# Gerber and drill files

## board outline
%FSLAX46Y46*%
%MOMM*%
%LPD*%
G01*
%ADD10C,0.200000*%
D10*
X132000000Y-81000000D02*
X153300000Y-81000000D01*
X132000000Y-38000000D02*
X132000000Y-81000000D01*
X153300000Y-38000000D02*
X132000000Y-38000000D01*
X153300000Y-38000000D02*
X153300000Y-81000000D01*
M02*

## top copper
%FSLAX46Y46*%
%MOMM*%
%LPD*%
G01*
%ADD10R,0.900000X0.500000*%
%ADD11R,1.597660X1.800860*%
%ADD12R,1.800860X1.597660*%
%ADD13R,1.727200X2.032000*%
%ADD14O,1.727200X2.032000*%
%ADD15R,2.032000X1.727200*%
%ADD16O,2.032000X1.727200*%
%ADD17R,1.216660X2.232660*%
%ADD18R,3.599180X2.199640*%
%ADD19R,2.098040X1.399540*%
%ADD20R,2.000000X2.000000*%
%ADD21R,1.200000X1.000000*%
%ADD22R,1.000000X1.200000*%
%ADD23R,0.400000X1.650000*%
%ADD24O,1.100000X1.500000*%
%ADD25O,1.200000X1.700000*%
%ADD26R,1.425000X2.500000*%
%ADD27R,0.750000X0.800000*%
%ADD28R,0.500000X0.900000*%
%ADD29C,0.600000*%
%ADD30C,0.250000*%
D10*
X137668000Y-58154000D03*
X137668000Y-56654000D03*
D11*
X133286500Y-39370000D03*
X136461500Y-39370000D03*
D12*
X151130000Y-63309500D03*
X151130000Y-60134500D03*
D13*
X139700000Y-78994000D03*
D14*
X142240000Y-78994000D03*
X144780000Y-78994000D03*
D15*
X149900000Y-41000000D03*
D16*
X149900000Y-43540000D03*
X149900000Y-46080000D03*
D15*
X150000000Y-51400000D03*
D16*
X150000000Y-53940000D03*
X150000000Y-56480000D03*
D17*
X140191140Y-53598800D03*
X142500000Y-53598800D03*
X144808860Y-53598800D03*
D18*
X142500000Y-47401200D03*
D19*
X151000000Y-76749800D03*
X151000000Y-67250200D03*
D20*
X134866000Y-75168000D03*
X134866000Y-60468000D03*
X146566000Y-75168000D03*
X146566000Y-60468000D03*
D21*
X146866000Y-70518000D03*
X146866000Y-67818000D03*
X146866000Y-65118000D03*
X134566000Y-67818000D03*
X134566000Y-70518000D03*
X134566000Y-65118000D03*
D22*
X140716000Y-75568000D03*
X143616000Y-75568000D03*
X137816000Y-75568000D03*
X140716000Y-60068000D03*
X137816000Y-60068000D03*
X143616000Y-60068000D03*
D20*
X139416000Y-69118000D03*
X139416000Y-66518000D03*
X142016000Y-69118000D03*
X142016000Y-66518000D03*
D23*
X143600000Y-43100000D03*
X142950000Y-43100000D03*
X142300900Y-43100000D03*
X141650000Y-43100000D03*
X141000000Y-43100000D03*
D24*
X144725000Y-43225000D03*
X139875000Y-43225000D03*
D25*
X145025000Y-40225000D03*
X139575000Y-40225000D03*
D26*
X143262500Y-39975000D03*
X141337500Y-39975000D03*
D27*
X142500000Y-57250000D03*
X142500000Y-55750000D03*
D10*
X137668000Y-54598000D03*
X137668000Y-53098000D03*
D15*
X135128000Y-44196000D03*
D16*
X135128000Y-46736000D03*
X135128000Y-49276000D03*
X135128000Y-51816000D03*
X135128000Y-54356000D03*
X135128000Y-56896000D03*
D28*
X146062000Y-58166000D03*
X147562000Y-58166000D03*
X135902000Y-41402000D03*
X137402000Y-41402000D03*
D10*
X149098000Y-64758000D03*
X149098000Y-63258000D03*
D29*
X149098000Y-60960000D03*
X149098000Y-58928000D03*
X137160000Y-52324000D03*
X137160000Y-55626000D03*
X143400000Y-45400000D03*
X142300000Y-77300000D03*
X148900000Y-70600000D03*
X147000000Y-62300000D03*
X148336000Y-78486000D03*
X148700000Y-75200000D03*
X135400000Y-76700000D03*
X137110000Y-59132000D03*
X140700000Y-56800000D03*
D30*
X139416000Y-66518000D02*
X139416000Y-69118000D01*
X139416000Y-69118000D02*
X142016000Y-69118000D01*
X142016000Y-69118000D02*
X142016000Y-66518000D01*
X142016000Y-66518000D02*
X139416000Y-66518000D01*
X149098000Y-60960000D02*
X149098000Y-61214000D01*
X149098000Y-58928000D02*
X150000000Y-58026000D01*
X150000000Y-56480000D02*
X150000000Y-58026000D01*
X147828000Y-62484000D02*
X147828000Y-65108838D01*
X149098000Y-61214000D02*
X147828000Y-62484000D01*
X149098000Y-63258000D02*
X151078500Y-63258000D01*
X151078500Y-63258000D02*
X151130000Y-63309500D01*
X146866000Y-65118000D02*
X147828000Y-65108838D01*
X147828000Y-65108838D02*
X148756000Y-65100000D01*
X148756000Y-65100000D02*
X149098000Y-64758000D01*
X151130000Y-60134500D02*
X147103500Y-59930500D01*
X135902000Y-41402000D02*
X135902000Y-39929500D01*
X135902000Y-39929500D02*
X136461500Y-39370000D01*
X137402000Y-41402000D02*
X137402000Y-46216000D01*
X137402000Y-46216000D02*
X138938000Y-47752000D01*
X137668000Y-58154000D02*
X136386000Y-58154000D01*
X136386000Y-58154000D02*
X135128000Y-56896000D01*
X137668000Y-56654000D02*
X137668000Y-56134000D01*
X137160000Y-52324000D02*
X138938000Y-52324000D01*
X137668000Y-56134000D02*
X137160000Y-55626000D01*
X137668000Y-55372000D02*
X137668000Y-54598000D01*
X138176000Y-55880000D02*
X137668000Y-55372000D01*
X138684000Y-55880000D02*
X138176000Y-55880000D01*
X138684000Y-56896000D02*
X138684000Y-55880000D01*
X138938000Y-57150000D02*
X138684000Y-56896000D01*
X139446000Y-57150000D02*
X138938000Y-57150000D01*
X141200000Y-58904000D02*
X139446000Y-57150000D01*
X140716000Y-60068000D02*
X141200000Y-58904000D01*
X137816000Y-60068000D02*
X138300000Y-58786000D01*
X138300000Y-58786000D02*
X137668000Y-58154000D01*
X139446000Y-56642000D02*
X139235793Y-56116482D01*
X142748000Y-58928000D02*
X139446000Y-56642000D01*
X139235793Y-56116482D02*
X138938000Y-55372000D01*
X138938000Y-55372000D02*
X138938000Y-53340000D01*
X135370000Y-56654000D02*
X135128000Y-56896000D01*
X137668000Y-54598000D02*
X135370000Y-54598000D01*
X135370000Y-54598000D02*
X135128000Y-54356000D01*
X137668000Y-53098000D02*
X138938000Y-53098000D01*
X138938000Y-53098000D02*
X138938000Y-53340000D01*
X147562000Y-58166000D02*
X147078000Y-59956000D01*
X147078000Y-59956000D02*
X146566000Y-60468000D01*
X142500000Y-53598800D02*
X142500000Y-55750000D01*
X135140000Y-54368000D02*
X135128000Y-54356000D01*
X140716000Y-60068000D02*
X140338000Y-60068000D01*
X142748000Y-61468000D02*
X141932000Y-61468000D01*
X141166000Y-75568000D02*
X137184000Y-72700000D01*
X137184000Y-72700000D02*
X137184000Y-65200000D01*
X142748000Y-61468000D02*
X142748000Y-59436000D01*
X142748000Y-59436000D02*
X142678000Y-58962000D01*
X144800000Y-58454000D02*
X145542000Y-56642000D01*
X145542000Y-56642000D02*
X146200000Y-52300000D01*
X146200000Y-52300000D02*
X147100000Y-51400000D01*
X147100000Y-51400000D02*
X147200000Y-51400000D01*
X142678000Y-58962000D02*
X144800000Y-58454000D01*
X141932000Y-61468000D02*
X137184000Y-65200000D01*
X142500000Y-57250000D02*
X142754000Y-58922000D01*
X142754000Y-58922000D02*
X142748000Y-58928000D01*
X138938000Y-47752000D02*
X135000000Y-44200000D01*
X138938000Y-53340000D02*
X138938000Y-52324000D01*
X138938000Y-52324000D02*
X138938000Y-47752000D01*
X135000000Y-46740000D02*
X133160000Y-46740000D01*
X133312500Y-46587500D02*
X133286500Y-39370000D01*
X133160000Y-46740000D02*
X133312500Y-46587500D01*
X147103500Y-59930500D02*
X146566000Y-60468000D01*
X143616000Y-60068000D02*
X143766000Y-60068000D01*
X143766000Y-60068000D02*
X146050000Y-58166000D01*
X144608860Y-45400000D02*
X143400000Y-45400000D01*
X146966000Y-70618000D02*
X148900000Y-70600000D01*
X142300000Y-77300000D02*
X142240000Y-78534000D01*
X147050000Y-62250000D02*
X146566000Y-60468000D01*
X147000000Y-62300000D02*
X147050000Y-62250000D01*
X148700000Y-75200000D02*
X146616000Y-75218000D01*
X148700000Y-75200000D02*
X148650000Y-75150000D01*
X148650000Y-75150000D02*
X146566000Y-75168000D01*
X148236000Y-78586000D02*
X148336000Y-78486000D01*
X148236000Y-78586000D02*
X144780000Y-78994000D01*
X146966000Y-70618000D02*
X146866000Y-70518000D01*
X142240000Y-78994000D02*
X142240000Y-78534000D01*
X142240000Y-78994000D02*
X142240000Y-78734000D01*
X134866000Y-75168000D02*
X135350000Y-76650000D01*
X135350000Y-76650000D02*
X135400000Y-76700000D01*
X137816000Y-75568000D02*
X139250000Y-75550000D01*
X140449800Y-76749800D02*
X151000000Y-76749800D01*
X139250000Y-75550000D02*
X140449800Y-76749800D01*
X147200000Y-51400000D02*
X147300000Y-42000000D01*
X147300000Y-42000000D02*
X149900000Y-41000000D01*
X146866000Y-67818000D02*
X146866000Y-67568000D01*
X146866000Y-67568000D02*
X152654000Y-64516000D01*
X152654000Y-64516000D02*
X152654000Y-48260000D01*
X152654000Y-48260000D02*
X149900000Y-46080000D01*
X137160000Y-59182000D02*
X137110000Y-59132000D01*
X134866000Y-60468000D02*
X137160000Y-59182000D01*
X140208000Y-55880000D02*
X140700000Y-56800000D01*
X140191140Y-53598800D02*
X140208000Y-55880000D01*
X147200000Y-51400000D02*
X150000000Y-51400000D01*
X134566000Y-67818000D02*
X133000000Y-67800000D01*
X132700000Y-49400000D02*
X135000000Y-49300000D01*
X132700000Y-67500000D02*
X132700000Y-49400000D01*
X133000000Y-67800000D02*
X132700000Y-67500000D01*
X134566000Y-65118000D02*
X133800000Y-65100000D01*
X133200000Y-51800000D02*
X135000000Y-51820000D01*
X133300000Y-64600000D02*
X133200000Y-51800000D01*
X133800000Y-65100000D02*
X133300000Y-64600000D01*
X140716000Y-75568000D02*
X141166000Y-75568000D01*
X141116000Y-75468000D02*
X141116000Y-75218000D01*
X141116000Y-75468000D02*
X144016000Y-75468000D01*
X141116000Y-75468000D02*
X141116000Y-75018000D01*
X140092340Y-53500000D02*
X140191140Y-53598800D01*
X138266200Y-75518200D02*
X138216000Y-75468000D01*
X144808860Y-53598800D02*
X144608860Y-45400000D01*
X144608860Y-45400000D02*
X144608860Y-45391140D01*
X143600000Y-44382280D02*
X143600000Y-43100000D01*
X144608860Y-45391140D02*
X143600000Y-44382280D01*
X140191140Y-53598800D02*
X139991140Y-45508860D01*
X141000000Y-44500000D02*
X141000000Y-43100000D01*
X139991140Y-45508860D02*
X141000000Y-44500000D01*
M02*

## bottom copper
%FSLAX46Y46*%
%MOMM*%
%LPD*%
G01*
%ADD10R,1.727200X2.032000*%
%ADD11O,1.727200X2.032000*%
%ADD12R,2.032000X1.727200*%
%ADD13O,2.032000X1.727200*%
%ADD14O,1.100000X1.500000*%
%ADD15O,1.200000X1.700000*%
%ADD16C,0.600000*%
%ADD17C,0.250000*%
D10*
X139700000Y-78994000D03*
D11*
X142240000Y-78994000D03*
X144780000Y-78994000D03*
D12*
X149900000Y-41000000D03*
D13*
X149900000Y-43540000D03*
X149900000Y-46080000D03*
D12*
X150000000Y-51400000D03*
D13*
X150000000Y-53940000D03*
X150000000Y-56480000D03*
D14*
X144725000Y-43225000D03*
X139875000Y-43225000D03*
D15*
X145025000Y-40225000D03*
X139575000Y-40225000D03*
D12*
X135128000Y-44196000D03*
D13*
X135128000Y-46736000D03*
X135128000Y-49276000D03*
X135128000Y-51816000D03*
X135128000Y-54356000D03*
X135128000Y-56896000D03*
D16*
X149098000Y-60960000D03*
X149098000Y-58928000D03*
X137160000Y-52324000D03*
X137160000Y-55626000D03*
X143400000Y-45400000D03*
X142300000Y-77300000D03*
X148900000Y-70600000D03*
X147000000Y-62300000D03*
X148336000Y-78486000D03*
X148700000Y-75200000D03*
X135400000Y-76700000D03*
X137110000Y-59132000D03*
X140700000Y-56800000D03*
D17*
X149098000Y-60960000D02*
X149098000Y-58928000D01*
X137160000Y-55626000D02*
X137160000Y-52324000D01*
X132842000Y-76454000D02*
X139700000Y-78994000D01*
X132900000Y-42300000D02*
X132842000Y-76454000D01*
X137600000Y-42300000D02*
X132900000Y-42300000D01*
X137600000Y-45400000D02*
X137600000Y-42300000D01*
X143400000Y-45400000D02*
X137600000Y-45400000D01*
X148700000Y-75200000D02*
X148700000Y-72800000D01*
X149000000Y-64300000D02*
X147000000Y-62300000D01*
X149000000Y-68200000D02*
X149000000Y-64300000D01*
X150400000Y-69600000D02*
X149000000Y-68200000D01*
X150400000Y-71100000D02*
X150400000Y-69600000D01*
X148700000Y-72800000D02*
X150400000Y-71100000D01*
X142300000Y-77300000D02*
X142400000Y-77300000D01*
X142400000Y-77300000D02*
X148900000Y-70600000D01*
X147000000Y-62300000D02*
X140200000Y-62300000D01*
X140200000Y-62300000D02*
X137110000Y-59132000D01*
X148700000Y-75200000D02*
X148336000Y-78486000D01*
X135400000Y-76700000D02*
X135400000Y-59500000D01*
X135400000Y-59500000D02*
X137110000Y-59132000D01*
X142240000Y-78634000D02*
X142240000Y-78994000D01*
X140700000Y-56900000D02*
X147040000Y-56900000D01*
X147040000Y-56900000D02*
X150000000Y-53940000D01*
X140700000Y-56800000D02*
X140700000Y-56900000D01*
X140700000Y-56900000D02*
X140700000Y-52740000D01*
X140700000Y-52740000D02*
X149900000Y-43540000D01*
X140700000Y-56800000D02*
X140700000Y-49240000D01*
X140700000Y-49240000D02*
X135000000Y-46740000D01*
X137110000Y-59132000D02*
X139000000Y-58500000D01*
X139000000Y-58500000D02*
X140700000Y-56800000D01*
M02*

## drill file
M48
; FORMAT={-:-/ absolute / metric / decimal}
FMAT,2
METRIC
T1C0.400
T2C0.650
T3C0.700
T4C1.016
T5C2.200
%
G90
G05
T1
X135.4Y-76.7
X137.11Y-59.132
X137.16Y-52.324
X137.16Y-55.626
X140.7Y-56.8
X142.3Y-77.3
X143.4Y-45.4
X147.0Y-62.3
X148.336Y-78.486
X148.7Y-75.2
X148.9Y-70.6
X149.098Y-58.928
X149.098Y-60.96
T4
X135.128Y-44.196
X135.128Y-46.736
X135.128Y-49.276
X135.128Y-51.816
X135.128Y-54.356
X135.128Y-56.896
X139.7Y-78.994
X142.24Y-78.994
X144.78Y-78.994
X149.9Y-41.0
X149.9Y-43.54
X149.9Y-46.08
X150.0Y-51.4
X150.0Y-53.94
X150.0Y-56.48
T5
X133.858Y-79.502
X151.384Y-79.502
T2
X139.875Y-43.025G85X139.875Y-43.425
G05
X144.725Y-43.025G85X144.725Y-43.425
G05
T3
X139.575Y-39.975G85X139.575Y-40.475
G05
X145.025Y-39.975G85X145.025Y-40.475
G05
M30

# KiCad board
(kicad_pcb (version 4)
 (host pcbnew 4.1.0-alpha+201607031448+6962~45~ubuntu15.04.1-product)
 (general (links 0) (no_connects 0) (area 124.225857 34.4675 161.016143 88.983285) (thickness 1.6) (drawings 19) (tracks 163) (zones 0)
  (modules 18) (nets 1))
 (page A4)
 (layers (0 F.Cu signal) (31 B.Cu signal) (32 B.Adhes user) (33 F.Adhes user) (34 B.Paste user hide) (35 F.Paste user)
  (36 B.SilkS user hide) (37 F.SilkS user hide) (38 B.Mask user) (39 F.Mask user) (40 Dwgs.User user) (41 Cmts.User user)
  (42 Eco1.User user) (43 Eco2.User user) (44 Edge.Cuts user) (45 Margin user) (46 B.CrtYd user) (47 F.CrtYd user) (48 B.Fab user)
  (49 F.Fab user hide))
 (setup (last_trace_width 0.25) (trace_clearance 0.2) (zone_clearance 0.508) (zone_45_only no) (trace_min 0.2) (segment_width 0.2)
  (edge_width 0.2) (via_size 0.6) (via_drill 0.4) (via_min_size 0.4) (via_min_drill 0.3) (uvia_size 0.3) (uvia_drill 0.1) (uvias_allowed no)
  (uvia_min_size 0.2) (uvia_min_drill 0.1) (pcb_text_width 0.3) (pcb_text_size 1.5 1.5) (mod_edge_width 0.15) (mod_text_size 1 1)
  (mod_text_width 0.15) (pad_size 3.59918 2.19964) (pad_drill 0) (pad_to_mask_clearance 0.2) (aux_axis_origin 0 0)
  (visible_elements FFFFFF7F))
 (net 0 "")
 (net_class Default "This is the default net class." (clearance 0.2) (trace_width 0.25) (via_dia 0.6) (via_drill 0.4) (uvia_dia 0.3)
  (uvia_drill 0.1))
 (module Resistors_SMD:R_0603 (layer F.Cu) (at 137.668 57.404 90)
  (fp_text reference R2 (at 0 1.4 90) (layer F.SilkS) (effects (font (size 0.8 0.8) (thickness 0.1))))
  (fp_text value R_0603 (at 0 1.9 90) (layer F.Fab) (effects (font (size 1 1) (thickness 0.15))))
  (pad 1 smd rect (at -0.75 0 90) (size 0.5 0.9) (layers F.Cu F.Paste F.Mask))
  (pad 2 smd rect (at 0.75 0 90) (size 0.5 0.9) (layers F.Cu F.Paste F.Mask)))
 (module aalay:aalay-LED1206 (layer F.Cu) (at 134.874 39.37)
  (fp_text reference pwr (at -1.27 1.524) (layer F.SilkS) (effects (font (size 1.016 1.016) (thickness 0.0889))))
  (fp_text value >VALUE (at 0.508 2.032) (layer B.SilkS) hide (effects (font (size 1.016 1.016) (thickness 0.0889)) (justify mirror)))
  (pad A smd rect (at -1.5875 0) (size 1.59766 1.80086) (layers F.Cu F.Paste F.Mask))
  (pad K smd rect (at 1.5875 0) (size 1.59766 1.80086) (layers F.Cu F.Paste F.Mask)))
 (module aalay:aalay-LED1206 (layer F.Cu) (at 151.13 61.722 90)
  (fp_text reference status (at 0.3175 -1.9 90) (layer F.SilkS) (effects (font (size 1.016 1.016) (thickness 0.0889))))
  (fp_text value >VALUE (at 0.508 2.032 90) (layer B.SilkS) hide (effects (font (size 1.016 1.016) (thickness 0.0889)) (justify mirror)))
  (pad A smd rect (at -1.5875 0 90) (size 1.59766 1.80086) (layers F.Cu F.Paste F.Mask))
  (pad K smd rect (at 1.5875 0 90) (size 1.59766 1.80086) (layers F.Cu F.Paste F.Mask)))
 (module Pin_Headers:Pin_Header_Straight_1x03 (layer F.Cu) (at 139.7 78.994 90)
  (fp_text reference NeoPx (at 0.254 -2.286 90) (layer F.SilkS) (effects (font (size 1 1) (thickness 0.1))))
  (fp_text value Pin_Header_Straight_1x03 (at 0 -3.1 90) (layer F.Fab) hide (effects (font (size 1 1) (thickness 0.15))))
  (pad 1 thru_hole rect (at 0 0 90) (size 2.032 1.7272) (drill 1.016) (layers *.Cu *.Mask F.SilkS))
  (pad 2 thru_hole oval (at 0 2.54 90) (size 2.032 1.7272) (drill 1.016) (layers *.Cu *.Mask F.SilkS))
  (pad 3 thru_hole oval (at 0 5.08 90) (size 2.032 1.7272) (drill 1.016) (layers *.Cu *.Mask F.SilkS)))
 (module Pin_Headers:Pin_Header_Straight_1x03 (layer F.Cu) (at 149.9 41)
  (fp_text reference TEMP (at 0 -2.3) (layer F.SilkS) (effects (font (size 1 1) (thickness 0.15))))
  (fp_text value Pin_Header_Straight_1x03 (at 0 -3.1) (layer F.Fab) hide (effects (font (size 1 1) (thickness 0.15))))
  (pad 1 thru_hole rect (at 0 0) (size 2.032 1.7272) (drill 1.016) (layers *.Cu *.Mask F.SilkS))
  (pad 2 thru_hole oval (at 0 2.54) (size 2.032 1.7272) (drill 1.016) (layers *.Cu *.Mask F.SilkS))
  (pad 3 thru_hole oval (at 0 5.08) (size 2.032 1.7272) (drill 1.016) (layers *.Cu *.Mask F.SilkS)))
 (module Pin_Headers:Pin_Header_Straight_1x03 (layer F.Cu) (at 150 51.4)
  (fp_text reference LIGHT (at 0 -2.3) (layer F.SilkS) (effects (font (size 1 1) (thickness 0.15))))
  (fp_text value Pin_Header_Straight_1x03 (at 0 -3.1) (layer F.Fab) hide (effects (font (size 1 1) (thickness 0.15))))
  (pad 1 thru_hole rect (at 0 0) (size 2.032 1.7272) (drill 1.016) (layers *.Cu *.Mask F.SilkS))
  (pad 2 thru_hole oval (at 0 2.54) (size 2.032 1.7272) (drill 1.016) (layers *.Cu *.Mask F.SilkS))
  (pad 3 thru_hole oval (at 0 5.08) (size 2.032 1.7272) (drill 1.016) (layers *.Cu *.Mask F.SilkS)))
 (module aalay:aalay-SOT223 (layer F.Cu) (at 142.5 50.5)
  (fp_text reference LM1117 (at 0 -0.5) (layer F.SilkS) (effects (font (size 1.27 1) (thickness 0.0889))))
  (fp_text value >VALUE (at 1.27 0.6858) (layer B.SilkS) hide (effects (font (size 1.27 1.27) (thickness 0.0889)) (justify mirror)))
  (pad GND smd rect (at -2.30886 3.0988) (size 1.21666 2.23266) (layers F.Cu F.Paste F.Mask))
  (pad OUT smd rect (at 0 3.0988) (size 1.21666 2.23266) (layers F.Cu F.Paste F.Mask))
  (pad IN smd rect (at 2.30886 3.0988) (size 1.21666 2.23266) (layers F.Cu F.Paste F.Mask))
  (pad OUT smd rect (at 0 -3.0988) (size 3.59918 2.19964) (layers F.Cu F.Paste F.Mask)))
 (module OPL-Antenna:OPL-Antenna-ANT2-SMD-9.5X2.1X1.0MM (layer F.Cu) (at 151 72 90)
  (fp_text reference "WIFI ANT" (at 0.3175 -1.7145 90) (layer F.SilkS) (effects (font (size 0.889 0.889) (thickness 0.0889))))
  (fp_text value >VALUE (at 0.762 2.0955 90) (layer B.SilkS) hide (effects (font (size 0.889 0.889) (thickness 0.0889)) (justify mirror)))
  (pad 1 smd rect (at -4.7498 0 90) (size 1.39954 2.09804) (layers F.Cu F.Paste F.Mask))
  (pad 2 smd rect (at 4.7498 0 90) (size 1.39954 2.09804) (layers F.Cu F.Paste F.Mask)))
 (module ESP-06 (layer F.Cu) (at 140.716 67.818 90)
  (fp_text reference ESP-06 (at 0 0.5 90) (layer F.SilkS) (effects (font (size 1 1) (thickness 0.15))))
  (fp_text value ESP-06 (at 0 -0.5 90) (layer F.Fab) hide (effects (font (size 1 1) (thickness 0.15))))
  (pad G smd rect (at -7.35 -5.85 90) (size 2 2) (layers F.Cu F.Paste F.Mask))
  (pad G smd rect (at 7.35 -5.85 90) (size 2 2) (layers F.Cu F.Paste F.Mask))
  (pad G smd rect (at -7.35 5.85 90) (size 2 2) (layers F.Cu F.Paste F.Mask))
  (pad G smd rect (at 7.35 5.85 90) (size 2 2) (layers F.Cu F.Paste F.Mask))
  (pad GP14 smd rect (at -2.7 6.15 90) (size 1 1.2) (layers F.Cu F.Paste F.Mask))
  (pad GP13 smd rect (at 0 6.15 90) (size 1 1.2) (layers F.Cu F.Paste F.Mask))
  (pad GP12 smd rect (at 2.7 6.15 90) (size 1 1.2) (layers F.Cu F.Paste F.Mask))
  (pad TX smd rect (at 0 -6.15 90) (size 1 1.2) (layers F.Cu F.Paste F.Mask))
  (pad GP16 smd rect (at -2.7 -6.15 90) (size 1 1.2) (layers F.Cu F.Paste F.Mask))
  (pad RX smd rect (at 2.7 -6.15 90) (size 1 1.2) (layers F.Cu F.Paste F.Mask))
  (pad 3.3 smd rect (at -7.75 0 90) (size 1.2 1) (layers F.Cu F.Paste F.Mask))
  (pad CHPD smd rect (at -7.75 2.9 90) (size 1.2 1) (layers F.Cu F.Paste F.Mask))
  (pad ANT smd rect (at -7.75 -2.9 90) (size 1.2 1) (layers F.Cu F.Paste F.Mask))
  (pad GP2 smd rect (at 7.75 0 90) (size 1.2 1) (layers F.Cu F.Paste F.Mask))
  (pad GP0 smd rect (at 7.75 -2.9 90) (size 1.2 1) (layers F.Cu F.Paste F.Mask))
  (pad GP15 smd rect (at 7.75 2.9 90) (size 1.2 1) (layers F.Cu F.Paste F.Mask))
  (pad Gx smd rect (at -1.3 -1.3 90) (size 2 2) (layers F.Cu F.Paste F.Mask))
  (pad Gx smd rect (at 1.3 -1.3 90) (size 2 2) (layers F.Cu F.Paste F.Mask))
  (pad Gx smd rect (at -1.3 1.3 90) (size 2 2) (layers F.Cu F.Paste F.Mask))
  (pad Gx smd rect (at 1.3 1.3 90) (size 2 2) (layers F.Cu F.Paste F.Mask)))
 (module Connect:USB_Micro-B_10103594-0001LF (layer F.Cu) (at 142.3 41.6 180)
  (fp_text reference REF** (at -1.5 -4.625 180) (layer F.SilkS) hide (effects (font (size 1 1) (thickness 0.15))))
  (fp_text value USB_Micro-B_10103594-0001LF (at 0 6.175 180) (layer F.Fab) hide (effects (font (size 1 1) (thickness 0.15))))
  (pad +5 smd rect (at -1.3 -1.5 270) (size 1.65 0.4) (layers F.Cu F.Paste F.Mask))
  (pad D- smd rect (at -0.65 -1.5 270) (size 1.65 0.4) (layers F.Cu F.Paste F.Mask))
  (pad D+ smd rect (at -0.0009 -1.5 270) (size 1.65 0.4) (layers F.Cu F.Paste F.Mask))
  (pad ID smd rect (at 0.65 -1.5 270) (size 1.65 0.4) (layers F.Cu F.Paste F.Mask))
  (pad GND smd rect (at 1.3 -1.5 270) (size 1.65 0.4) (layers F.Cu F.Paste F.Mask))
  (pad 6 thru_hole oval (at -2.425 -1.625 270) (size 1.5 1.1) (drill oval 1.05 0.65) (layers *.Cu *.Mask F.SilkS))
  (pad 6 thru_hole oval (at 2.425 -1.625 270) (size 1.5 1.1) (drill oval 1.05 0.65) (layers *.Cu *.Mask F.SilkS))
  (pad 6 thru_hole oval (at -2.725 1.375 270) (size 1.7 1.2) (drill oval 1.2 0.7) (layers *.Cu *.Mask F.SilkS))
  (pad 6 thru_hole oval (at 2.725 1.375 270) (size 1.7 1.2) (drill oval 1.2 0.7) (layers *.Cu *.Mask F.SilkS))
  (pad 6 smd rect (at -0.9625 1.625 270) (size 2.5 1.425) (layers F.Cu F.Paste F.Mask))
  (pad 6 smd rect (at 0.9625 1.625 270) (size 2.5 1.425) (layers F.Cu F.Paste F.Mask)))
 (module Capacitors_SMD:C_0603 (layer F.Cu) (at 142.5 56.5 90)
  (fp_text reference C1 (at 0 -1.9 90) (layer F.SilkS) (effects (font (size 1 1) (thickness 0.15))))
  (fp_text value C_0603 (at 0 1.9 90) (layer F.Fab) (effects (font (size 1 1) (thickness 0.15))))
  (pad 1 smd rect (at -0.75 0 90) (size 0.8 0.75) (layers F.Cu F.Paste F.Mask))
  (pad 2 smd rect (at 0.75 0 90) (size 0.8 0.75) (layers F.Cu F.Paste F.Mask)))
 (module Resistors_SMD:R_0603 (layer F.Cu) (at 137.668 53.848 90)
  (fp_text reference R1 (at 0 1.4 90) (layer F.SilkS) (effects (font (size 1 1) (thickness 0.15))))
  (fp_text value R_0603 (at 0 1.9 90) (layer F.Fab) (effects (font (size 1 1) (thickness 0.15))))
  (pad 1 smd rect (at -0.75 0 90) (size 0.5 0.9) (layers F.Cu F.Paste F.Mask))
  (pad 2 smd rect (at 0.75 0 90) (size 0.5 0.9) (layers F.Cu F.Paste F.Mask)))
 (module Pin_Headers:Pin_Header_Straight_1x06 (layer F.Cu) (at 135.128 44.196)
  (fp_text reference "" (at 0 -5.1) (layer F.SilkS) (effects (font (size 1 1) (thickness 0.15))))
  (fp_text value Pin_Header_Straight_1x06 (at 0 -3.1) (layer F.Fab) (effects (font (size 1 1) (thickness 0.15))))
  (pad 1 thru_hole rect (at 0 0) (size 2.032 1.7272) (drill 1.016) (layers *.Cu *.Mask F.SilkS))
  (pad 2 thru_hole oval (at 0 2.54) (size 2.032 1.7272) (drill 1.016) (layers *.Cu *.Mask F.SilkS))
  (pad 3 thru_hole oval (at 0 5.08) (size 2.032 1.7272) (drill 1.016) (layers *.Cu *.Mask F.SilkS))
  (pad 4 thru_hole oval (at 0 7.62) (size 2.032 1.7272) (drill 1.016) (layers *.Cu *.Mask F.SilkS))
  (pad 5 thru_hole oval (at 0 10.16) (size 2.032 1.7272) (drill 1.016) (layers *.Cu *.Mask F.SilkS))
  (pad 6 thru_hole oval (at 0 12.7) (size 2.032 1.7272) (drill 1.016) (layers *.Cu *.Mask F.SilkS)))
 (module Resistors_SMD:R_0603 (layer F.Cu) (at 146.812 58.166)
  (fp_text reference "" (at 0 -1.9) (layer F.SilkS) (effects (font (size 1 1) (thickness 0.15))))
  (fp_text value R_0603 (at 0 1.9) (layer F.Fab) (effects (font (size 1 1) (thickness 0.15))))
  (pad 1 smd rect (at -0.75 0) (size 0.5 0.9) (layers F.Cu F.Paste F.Mask))
  (pad 2 smd rect (at 0.75 0) (size 0.5 0.9) (layers F.Cu F.Paste F.Mask)))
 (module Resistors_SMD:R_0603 (layer F.Cu) (at 136.652 41.402)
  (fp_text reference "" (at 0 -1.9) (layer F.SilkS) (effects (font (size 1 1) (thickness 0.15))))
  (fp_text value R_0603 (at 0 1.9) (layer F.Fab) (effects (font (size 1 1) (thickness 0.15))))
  (pad 1 smd rect (at -0.75 0) (size 0.5 0.9) (layers F.Cu F.Paste F.Mask))
  (pad 2 smd rect (at 0.75 0) (size 0.5 0.9) (layers F.Cu F.Paste F.Mask)))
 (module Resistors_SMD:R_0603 (layer F.Cu) (at 149.098 64.008 90)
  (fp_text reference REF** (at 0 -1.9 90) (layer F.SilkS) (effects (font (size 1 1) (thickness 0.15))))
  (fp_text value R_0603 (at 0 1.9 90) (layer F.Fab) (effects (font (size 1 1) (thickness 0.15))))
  (pad 1 smd rect (at -0.75 0 90) (size 0.5 0.9) (layers F.Cu F.Paste F.Mask))
  (pad 2 smd rect (at 0.75 0 90) (size 0.5 0.9) (layers F.Cu F.Paste F.Mask)))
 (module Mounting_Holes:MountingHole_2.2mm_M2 (layer F.Cu) (at 133.858 79.502)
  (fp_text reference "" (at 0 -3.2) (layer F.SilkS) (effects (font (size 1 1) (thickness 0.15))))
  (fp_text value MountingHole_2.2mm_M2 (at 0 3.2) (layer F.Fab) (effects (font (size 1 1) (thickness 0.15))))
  (pad 1 np_thru_hole circle (at 0 0) (size 2.2 2.2) (drill 2.2) (layers *.Cu *.Mask F.SilkS)))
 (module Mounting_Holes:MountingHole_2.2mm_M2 (layer F.Cu) (at 151.384 79.502)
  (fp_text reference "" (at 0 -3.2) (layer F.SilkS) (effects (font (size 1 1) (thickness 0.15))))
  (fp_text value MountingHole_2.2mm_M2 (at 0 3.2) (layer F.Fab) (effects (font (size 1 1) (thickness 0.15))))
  (pad 1 np_thru_hole circle (at 0 0) (size 2.2 2.2) (drill 2.2) (layers *.Cu *.Mask F.SilkS)))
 (gr_line (start 132 81) (end 153.3 81) (angle 90) (layer Edge.Cuts) (width 0.2))
 (gr_line (start 132 38) (end 132 81) (angle 90) (layer Edge.Cuts) (width 0.2))
 (gr_line (start 153.3 38) (end 132 38) (angle 90) (layer Edge.Cuts) (width 0.2))
 (gr_line (start 153.3 38) (end 153.3 81) (angle 90) (layer Edge.Cuts) (width 0.2))
 (segment (start 139.416 66.518) (end 139.416 69.118) (width 0.25) (layer F.Cu) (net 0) (status C00000))
 (segment (start 139.416 69.118) (end 142.016 69.118) (width 0.25) (layer F.Cu) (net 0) (status C00000))
 (segment (start 142.016 69.118) (end 142.016 66.518) (width 0.25) (layer F.Cu) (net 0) (status C00000))
 (segment (start 142.016 66.518) (end 139.416 66.518) (width 0.25) (layer F.Cu) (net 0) (status C00000))
 (segment (start 149.098 60.96) (end 149.098 61.214) (width 0.25) (layer F.Cu) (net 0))
 (via (at 149.098 60.96) (size 0.6) (drill 0.4) (layers F.Cu B.Cu) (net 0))
 (segment (start 149.098 60.96) (end 149.098 58.928) (width 0.25) (layer B.Cu) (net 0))
 (via (at 149.098 58.928) (size 0.6) (drill 0.4) (layers F.Cu B.Cu) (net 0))
 (segment (start 149.098 58.928) (end 150 58.026) (width 0.25) (layer F.Cu) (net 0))
 (segment (start 150 56.48) (end 150 58.026) (width 0.25) (layer F.Cu) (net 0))
 (segment (start 147.828 62.484) (end 147.828 65.108838) (width 0.25) (layer F.Cu) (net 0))
 (segment (start 149.098 61.214) (end 147.828 62.484) (width 0.25) (layer F.Cu) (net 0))
 (segment (start 149.098 63.258) (end 151.0785 63.258) (width 0.25) (layer F.Cu) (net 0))
 (segment (start 151.0785 63.258) (end 151.13 63.3095) (width 0.25) (layer F.Cu) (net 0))
 (segment (start 146.866 65.118) (end 147.828 65.108838) (width 0.25) (layer F.Cu) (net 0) (status 10))
 (segment (start 147.828 65.108838) (end 148.756 65.1) (width 0.25) (layer F.Cu) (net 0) (status 10))
 (segment (start 148.756 65.1) (end 149.098 64.758) (width 0.25) (layer F.Cu) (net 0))
 (segment (start 151.13 60.1345) (end 147.1035 59.9305) (width 0.25) (layer F.Cu) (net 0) (status 20))
 (segment (start 135.902 41.402) (end 135.902 39.9295) (width 0.25) (layer F.Cu) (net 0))
 (segment (start 135.902 39.9295) (end 136.4615 39.37) (width 0.25) (layer F.Cu) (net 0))
 (segment (start 137.402 41.402) (end 137.402 46.216) (width 0.25) (layer F.Cu) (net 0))
 (segment (start 137.402 46.216) (end 138.938 47.752) (width 0.25) (layer F.Cu) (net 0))
 (segment (start 137.668 58.154) (end 136.386 58.154) (width 0.25) (layer F.Cu) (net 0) (status 10))
 (segment (start 136.386 58.154) (end 135.128 56.896) (width 0.25) (layer F.Cu) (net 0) (status 20))
 (segment (start 137.668 56.654) (end 137.668 56.134) (width 0.25) (layer F.Cu) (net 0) (status 10))
 (segment (start 137.16 52.324) (end 138.938 52.324) (width 0.25) (layer F.Cu) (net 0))
 (via (at 137.16 52.324) (size 0.6) (drill 0.4) (layers F.Cu B.Cu) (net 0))
 (segment (start 137.16 55.626) (end 137.16 52.324) (width 0.25) (layer B.Cu) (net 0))
 (via (at 137.16 55.626) (size 0.6) (drill 0.4) (layers F.Cu B.Cu) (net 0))
 (segment (start 137.668 56.134) (end 137.16 55.626) (width 0.25) (layer F.Cu) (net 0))
 (segment (start 137.668 55.372) (end 137.668 54.598) (width 0.25) (layer F.Cu) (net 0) (status 20))
 (segment (start 138.176 55.88) (end 137.668 55.372) (width 0.25) (layer F.Cu) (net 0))
 (segment (start 138.684 55.88) (end 138.176 55.88) (width 0.25) (layer F.Cu) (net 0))
 (segment (start 138.684 56.896) (end 138.684 55.88) (width 0.25) (layer F.Cu) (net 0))
 (segment (start 138.938 57.15) (end 138.684 56.896) (width 0.25) (layer F.Cu) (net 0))
 (segment (start 139.446 57.15) (end 138.938 57.15) (width 0.25) (layer F.Cu) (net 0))
 (segment (start 141.2 58.904) (end 139.446 57.15) (width 0.25) (layer F.Cu) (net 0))
 (segment (start 140.716 60.068) (end 141.2 58.904) (width 0.25) (layer F.Cu) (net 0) (status 10))
 (segment (start 137.816 60.068) (end 138.3 58.786) (width 0.25) (layer F.Cu) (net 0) (status 10))
 (segment (start 138.3 58.786) (end 137.668 58.154) (width 0.25) (layer F.Cu) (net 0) (status 20))
 (segment (start 139.446 56.642) (end 139.235793 56.116482) (width 0.25) (layer F.Cu) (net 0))
 (segment (start 142.748 58.928) (end 139.446 56.642) (width 0.25) (layer F.Cu) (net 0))
 (segment (start 139.235793 56.116482) (end 138.938 55.372) (width 0.25) (layer F.Cu) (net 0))
 (segment (start 138.938 55.372) (end 138.938 53.34) (width 0.25) (layer F.Cu) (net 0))
 (segment (start 135.37 56.654) (end 135.128 56.896) (width 0.25) (layer F.Cu) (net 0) (status 30))
 (segment (start 137.668 54.598) (end 135.37 54.598) (width 0.25) (layer F.Cu) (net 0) (status 30))
 (segment (start 135.37 54.598) (end 135.128 54.356) (width 0.25) (layer F.Cu) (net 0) (status 30))
 (segment (start 137.668 53.098) (end 138.938 53.098) (width 0.25) (layer F.Cu) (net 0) (status 10))
 (segment (start 138.938 53.098) (end 138.938 53.34) (width 0.25) (layer F.Cu) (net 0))
 (segment (start 147.562 58.166) (end 147.078 59.956) (width 0.25) (layer F.Cu) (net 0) (status 20))
 (segment (start 147.078 59.956) (end 146.566 60.468) (width 0.25) (layer F.Cu) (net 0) (status 30))
 (segment (start 142.5 53.5988) (end 142.5 55.75) (width 0.25) (layer F.Cu) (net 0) (status 30))
 (segment (start 135.14 54.368) (end 135.128 54.356) (width 0.25) (layer F.Cu) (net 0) (status 30))
 (segment (start 140.716 60.068) (end 140.338 60.068) (width 0.25) (layer F.Cu) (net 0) (status 30))
 (segment (start 142.748 61.468) (end 141.932 61.468) (width 0.25) (layer F.Cu) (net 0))
 (segment (start 141.166 75.568) (end 137.184 72.7) (width 0.25) (layer F.Cu) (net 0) (status 10))
 (segment (start 137.184 72.7) (end 137.184 65.2) (width 0.25) (layer F.Cu) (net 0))
 (segment (start 142.748 61.468) (end 142.748 59.436) (width 0.25) (layer F.Cu) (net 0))
 (segment (start 142.748 59.436) (end 142.678 58.962) (width 0.25) (layer F.Cu) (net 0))
 (segment (start 144.8 58.454) (end 145.542 56.642) (width 0.25) (layer F.Cu) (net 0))
 (segment (start 145.542 56.642) (end 146.2 52.3) (width 0.25) (layer F.Cu) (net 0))
 (segment (start 146.2 52.3) (end 147.1 51.4) (width 0.25) (layer F.Cu) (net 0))
 (segment (start 147.1 51.4) (end 147.2 51.4) (width 0.25) (layer F.Cu) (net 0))
 (segment (start 142.678 58.962) (end 144.8 58.454) (width 0.25) (layer F.Cu) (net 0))
 (segment (start 141.932 61.468) (end 137.184 65.2) (width 0.25) (layer F.Cu) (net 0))
 (segment (start 142.5 57.25) (end 142.754 58.922) (width 0.25) (layer F.Cu) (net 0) (status 10))
 (segment (start 142.754 58.922) (end 142.748 58.928) (width 0.25) (layer F.Cu) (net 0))
 (segment (start 138.938 47.752) (end 135 44.2) (width 0.25) (layer F.Cu) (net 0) (status 20))
 (segment (start 138.938 53.34) (end 138.938 52.324) (width 0.25) (layer F.Cu) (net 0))
 (segment (start 138.938 52.324) (end 138.938 47.752) (width 0.25) (layer F.Cu) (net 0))
 (segment (start 135 46.74) (end 133.16 46.74) (width 0.25) (layer F.Cu) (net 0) (status 10))
 (segment (start 133.3125 46.5875) (end 133.2865 39.37) (width 0.25) (layer F.Cu) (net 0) (status 20))
 (segment (start 133.16 46.74) (end 133.3125 46.5875) (width 0.25) (layer F.Cu) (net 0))
 (segment (start 147.1035 59.9305) (end 146.566 60.468) (width 0.25) (layer F.Cu) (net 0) (status 30))
 (segment (start 143.616 60.068) (end 143.766 60.068) (width 0.25) (layer F.Cu) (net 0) (status 30))
 (segment (start 143.766 60.068) (end 146.05 58.166) (width 0.25) (layer F.Cu) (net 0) (status 10))
 (segment (start 144.60886 45.4) (end 143.4 45.4) (width 0.25) (layer F.Cu) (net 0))
 (segment (start 132.842 76.454) (end 139.7 78.994) (width 0.25) (layer B.Cu) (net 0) (status 20))
 (segment (start 132.9 42.3) (end 132.842 76.454) (width 0.25) (layer B.Cu) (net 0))
 (segment (start 137.6 42.3) (end 132.9 42.3) (width 0.25) (layer B.Cu) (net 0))
 (segment (start 137.6 45.4) (end 137.6 42.3) (width 0.25) (layer B.Cu) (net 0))
 (segment (start 143.4 45.4) (end 137.6 45.4) (width 0.25) (layer B.Cu) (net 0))
 (via (at 143.4 45.4) (size 0.6) (drill 0.4) (layers F.Cu B.Cu) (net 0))
 (segment (start 148.7 75.2) (end 148.7 72.8) (width 0.25) (layer B.Cu) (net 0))
 (segment (start 149 64.3) (end 147 62.3) (width 0.25) (layer B.Cu) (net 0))
 (segment (start 149 68.2) (end 149 64.3) (width 0.25) (layer B.Cu) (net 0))
 (segment (start 150.4 69.6) (end 149 68.2) (width 0.25) (layer B.Cu) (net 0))
 (segment (start 150.4 71.1) (end 150.4 69.6) (width 0.25) (layer B.Cu) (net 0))
 (segment (start 148.7 72.8) (end 150.4 71.1) (width 0.25) (layer B.Cu) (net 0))
 (segment (start 146.966 70.618) (end 148.9 70.6) (width 0.25) (layer F.Cu) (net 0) (status 10))
 (segment (start 142.3 77.3) (end 142.4 77.3) (width 0.25) (layer B.Cu) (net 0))
 (via (at 142.3 77.3) (size 0.6) (drill 0.4) (layers F.Cu B.Cu) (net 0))
 (segment (start 142.3 77.3) (end 142.24 78.534) (width 0.25) (layer F.Cu) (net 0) (status 20))
 (via (at 148.9 70.6) (size 0.6) (drill 0.4) (layers F.Cu B.Cu) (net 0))
 (segment (start 142.4 77.3) (end 148.9 70.6) (width 0.25) (layer B.Cu) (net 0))
 (segment (start 147 62.3) (end 140.2 62.3) (width 0.25) (layer B.Cu) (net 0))
 (segment (start 140.2 62.3) (end 137.11 59.132) (width 0.25) (layer B.Cu) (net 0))
 (segment (start 147.05 62.25) (end 146.566 60.468) (width 0.25) (layer F.Cu) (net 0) (status 20))
 (via (at 147 62.3) (size 0.6) (drill 0.4) (layers F.Cu B.Cu) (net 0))
 (segment (start 147 62.3) (end 147.05 62.25) (width 0.25) (layer F.Cu) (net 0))
 (segment (start 148.7 75.2) (end 146.616 75.218) (width 0.25) (layer F.Cu) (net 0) (status 20))
 (segment (start 148.7 75.2) (end 148.65 75.15) (width 0.25) (layer F.Cu) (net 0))
 (segment (start 148.65 75.15) (end 146.566 75.168) (width 0.25) (layer F.Cu) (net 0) (status 20))
 (segment (start 148.7 75.2) (end 148.336 78.486) (width 0.25) (layer B.Cu) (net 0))
 (segment (start 148.236 78.586) (end 148.336 78.486) (width 0.25) (layer F.Cu) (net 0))
 (via (at 148.336 78.486) (size 0.6) (drill 0.4) (layers F.Cu B.Cu) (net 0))
 (segment (start 148.236 78.586) (end 144.78 78.994) (width 0.25) (layer F.Cu) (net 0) (status 20))
 (via (at 148.7 75.2) (size 0.6) (drill 0.4) (layers F.Cu B.Cu) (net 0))
 (segment (start 146.966 70.618) (end 146.866 70.518) (width 0.25) (layer F.Cu) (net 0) (status 30))
 (segment (start 142.24 78.994) (end 142.24 78.534) (width 0.25) (layer F.Cu) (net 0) (status 30))
 (segment (start 142.24 78.994) (end 142.24 78.734) (width 0.25) (layer F.Cu) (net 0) (status 30))
 (segment (start 135.4 76.7) (end 135.4 59.5) (width 0.25) (layer B.Cu) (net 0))
 (via (at 135.4 76.7) (size 0.6) (drill 0.4) (layers F.Cu B.Cu) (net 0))
 (segment (start 134.866 75.168) (end 135.35 76.65) (width 0.25) (layer F.Cu) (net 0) (status 10))
 (segment (start 135.35 76.65) (end 135.4 76.7) (width 0.25) (layer F.Cu) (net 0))
 (segment (start 135.4 59.5) (end 137.11 59.132) (width 0.25) (layer B.Cu) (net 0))
 (segment (start 142.24 78.634) (end 142.24 78.994) (width 0.25) (layer B.Cu) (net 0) (status 30))
 (segment (start 137.816 75.568) (end 139.25 75.55) (width 0.25) (layer F.Cu) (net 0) (status 10))
 (segment (start 140.4498 76.7498) (end 151 76.7498) (width 0.25) (layer F.Cu) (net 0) (status 20))
 (segment (start 139.25 75.55) (end 140.4498 76.7498) (width 0.25) (layer F.Cu) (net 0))
 (segment (start 147.2 51.4) (end 147.3 42) (width 0.25) (layer F.Cu) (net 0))
 (segment (start 147.3 42) (end 149.9 41) (width 0.25) (layer F.Cu) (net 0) (status 20))
 (segment (start 140.7 56.9) (end 147.04 56.9) (width 0.25) (layer B.Cu) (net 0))
 (segment (start 147.04 56.9) (end 150 53.94) (width 0.25) (layer B.Cu) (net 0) (status 20))
 (segment (start 146.866 67.818) (end 146.866 67.568) (width 0.25) (layer F.Cu) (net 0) (status 30))
 (segment (start 146.866 67.568) (end 152.654 64.516) (width 0.25) (layer F.Cu) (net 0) (status 10))
 (segment (start 152.654 64.516) (end 152.654 48.26) (width 0.25) (layer F.Cu) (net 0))
 (segment (start 152.654 48.26) (end 149.9 46.08) (width 0.25) (layer F.Cu) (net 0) (status 20))
 (segment (start 140.7 56.8) (end 140.7 56.9) (width 0.25) (layer B.Cu) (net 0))
 (segment (start 140.7 56.9) (end 140.7 52.74) (width 0.25) (layer B.Cu) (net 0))
 (segment (start 140.7 52.74) (end 149.9 43.54) (width 0.25) (layer B.Cu) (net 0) (status 20))
 (segment (start 140.7 56.8) (end 140.7 49.24) (width 0.25) (layer B.Cu) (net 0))
 (segment (start 140.7 49.24) (end 135 46.74) (width 0.25) (layer B.Cu) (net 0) (status 20))
 (segment (start 137.11 59.132) (end 139 58.5) (width 0.25) (layer B.Cu) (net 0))
 (segment (start 139 58.5) (end 140.7 56.8) (width 0.25) (layer B.Cu) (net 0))
 (segment (start 137.16 59.182) (end 137.11 59.132) (width 0.25) (layer F.Cu) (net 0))
 (via (at 137.11 59.132) (size 0.6) (drill 0.4) (layers F.Cu B.Cu) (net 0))
 (segment (start 134.866 60.468) (end 137.16 59.182) (width 0.25) (layer F.Cu) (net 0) (status 10))
 (segment (start 140.208 55.88) (end 140.7 56.8) (width 0.25) (layer F.Cu) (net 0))
 (via (at 140.7 56.8) (size 0.6) (drill 0.4) (layers F.Cu B.Cu) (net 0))
 (segment (start 140.19114 53.5988) (end 140.208 55.88) (width 0.25) (layer F.Cu) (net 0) (status 10))
 (segment (start 147.2 51.4) (end 150 51.4) (width 0.25) (layer F.Cu) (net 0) (status 20))
 (segment (start 134.566 67.818) (end 133 67.8) (width 0.25) (layer F.Cu) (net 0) (status 10))
 (segment (start 132.7 49.4) (end 135 49.3) (width 0.25) (layer F.Cu) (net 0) (status 20))
 (segment (start 132.7 67.5) (end 132.7 49.4) (width 0.25) (layer F.Cu) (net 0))
 (segment (start 133 67.8) (end 132.7 67.5) (width 0.25) (layer F.Cu) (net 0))
 (segment (start 134.566 65.118) (end 133.8 65.1) (width 0.25) (layer F.Cu) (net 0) (status 10))
 (segment (start 133.2 51.8) (end 135 51.82) (width 0.25) (layer F.Cu) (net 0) (status 20))
 (segment (start 133.3 64.6) (end 133.2 51.8) (width 0.25) (layer F.Cu) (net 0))
 (segment (start 133.8 65.1) (end 133.3 64.6) (width 0.25) (layer F.Cu) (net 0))
 (segment (start 140.716 75.568) (end 141.166 75.568) (width 0.25) (layer F.Cu) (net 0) (status 30))
 (segment (start 141.116 75.468) (end 141.116 75.218) (width 0.25) (layer F.Cu) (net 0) (status 30))
 (segment (start 141.116 75.468) (end 144.016 75.468) (width 0.25) (layer F.Cu) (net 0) (status 30))
 (segment (start 141.116 75.468) (end 141.116 75.018) (width 0.25) (layer F.Cu) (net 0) (status 30))
 (segment (start 140.09234 53.5) (end 140.19114 53.5988) (width 0.25) (layer F.Cu) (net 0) (status 30))
 (segment (start 138.2662 75.5182) (end 138.216 75.468) (width 0.25) (layer F.Cu) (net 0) (status 30))
 (segment (start 144.80886 53.5988) (end 144.60886 45.4) (width 0.25) (layer F.Cu) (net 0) (status 10))
 (segment (start 144.60886 45.4) (end 144.60886 45.39114) (width 0.25) (layer F.Cu) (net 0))
 (segment (start 143.6 44.38228) (end 143.6 43.1) (width 0.25) (layer F.Cu) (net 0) (status 20))
 (segment (start 144.60886 45.39114) (end 143.6 44.38228) (width 0.25) (layer F.Cu) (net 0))
 (segment (start 140.19114 53.5988) (end 139.99114 45.50886) (width 0.25) (layer F.Cu) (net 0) (status 10))
 (segment (start 141 44.5) (end 141 43.1) (width 0.25) (layer F.Cu) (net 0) (status 20))
 (segment (start 139.99114 45.50886) (end 141 44.5) (width 0.25) (layer F.Cu) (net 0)))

